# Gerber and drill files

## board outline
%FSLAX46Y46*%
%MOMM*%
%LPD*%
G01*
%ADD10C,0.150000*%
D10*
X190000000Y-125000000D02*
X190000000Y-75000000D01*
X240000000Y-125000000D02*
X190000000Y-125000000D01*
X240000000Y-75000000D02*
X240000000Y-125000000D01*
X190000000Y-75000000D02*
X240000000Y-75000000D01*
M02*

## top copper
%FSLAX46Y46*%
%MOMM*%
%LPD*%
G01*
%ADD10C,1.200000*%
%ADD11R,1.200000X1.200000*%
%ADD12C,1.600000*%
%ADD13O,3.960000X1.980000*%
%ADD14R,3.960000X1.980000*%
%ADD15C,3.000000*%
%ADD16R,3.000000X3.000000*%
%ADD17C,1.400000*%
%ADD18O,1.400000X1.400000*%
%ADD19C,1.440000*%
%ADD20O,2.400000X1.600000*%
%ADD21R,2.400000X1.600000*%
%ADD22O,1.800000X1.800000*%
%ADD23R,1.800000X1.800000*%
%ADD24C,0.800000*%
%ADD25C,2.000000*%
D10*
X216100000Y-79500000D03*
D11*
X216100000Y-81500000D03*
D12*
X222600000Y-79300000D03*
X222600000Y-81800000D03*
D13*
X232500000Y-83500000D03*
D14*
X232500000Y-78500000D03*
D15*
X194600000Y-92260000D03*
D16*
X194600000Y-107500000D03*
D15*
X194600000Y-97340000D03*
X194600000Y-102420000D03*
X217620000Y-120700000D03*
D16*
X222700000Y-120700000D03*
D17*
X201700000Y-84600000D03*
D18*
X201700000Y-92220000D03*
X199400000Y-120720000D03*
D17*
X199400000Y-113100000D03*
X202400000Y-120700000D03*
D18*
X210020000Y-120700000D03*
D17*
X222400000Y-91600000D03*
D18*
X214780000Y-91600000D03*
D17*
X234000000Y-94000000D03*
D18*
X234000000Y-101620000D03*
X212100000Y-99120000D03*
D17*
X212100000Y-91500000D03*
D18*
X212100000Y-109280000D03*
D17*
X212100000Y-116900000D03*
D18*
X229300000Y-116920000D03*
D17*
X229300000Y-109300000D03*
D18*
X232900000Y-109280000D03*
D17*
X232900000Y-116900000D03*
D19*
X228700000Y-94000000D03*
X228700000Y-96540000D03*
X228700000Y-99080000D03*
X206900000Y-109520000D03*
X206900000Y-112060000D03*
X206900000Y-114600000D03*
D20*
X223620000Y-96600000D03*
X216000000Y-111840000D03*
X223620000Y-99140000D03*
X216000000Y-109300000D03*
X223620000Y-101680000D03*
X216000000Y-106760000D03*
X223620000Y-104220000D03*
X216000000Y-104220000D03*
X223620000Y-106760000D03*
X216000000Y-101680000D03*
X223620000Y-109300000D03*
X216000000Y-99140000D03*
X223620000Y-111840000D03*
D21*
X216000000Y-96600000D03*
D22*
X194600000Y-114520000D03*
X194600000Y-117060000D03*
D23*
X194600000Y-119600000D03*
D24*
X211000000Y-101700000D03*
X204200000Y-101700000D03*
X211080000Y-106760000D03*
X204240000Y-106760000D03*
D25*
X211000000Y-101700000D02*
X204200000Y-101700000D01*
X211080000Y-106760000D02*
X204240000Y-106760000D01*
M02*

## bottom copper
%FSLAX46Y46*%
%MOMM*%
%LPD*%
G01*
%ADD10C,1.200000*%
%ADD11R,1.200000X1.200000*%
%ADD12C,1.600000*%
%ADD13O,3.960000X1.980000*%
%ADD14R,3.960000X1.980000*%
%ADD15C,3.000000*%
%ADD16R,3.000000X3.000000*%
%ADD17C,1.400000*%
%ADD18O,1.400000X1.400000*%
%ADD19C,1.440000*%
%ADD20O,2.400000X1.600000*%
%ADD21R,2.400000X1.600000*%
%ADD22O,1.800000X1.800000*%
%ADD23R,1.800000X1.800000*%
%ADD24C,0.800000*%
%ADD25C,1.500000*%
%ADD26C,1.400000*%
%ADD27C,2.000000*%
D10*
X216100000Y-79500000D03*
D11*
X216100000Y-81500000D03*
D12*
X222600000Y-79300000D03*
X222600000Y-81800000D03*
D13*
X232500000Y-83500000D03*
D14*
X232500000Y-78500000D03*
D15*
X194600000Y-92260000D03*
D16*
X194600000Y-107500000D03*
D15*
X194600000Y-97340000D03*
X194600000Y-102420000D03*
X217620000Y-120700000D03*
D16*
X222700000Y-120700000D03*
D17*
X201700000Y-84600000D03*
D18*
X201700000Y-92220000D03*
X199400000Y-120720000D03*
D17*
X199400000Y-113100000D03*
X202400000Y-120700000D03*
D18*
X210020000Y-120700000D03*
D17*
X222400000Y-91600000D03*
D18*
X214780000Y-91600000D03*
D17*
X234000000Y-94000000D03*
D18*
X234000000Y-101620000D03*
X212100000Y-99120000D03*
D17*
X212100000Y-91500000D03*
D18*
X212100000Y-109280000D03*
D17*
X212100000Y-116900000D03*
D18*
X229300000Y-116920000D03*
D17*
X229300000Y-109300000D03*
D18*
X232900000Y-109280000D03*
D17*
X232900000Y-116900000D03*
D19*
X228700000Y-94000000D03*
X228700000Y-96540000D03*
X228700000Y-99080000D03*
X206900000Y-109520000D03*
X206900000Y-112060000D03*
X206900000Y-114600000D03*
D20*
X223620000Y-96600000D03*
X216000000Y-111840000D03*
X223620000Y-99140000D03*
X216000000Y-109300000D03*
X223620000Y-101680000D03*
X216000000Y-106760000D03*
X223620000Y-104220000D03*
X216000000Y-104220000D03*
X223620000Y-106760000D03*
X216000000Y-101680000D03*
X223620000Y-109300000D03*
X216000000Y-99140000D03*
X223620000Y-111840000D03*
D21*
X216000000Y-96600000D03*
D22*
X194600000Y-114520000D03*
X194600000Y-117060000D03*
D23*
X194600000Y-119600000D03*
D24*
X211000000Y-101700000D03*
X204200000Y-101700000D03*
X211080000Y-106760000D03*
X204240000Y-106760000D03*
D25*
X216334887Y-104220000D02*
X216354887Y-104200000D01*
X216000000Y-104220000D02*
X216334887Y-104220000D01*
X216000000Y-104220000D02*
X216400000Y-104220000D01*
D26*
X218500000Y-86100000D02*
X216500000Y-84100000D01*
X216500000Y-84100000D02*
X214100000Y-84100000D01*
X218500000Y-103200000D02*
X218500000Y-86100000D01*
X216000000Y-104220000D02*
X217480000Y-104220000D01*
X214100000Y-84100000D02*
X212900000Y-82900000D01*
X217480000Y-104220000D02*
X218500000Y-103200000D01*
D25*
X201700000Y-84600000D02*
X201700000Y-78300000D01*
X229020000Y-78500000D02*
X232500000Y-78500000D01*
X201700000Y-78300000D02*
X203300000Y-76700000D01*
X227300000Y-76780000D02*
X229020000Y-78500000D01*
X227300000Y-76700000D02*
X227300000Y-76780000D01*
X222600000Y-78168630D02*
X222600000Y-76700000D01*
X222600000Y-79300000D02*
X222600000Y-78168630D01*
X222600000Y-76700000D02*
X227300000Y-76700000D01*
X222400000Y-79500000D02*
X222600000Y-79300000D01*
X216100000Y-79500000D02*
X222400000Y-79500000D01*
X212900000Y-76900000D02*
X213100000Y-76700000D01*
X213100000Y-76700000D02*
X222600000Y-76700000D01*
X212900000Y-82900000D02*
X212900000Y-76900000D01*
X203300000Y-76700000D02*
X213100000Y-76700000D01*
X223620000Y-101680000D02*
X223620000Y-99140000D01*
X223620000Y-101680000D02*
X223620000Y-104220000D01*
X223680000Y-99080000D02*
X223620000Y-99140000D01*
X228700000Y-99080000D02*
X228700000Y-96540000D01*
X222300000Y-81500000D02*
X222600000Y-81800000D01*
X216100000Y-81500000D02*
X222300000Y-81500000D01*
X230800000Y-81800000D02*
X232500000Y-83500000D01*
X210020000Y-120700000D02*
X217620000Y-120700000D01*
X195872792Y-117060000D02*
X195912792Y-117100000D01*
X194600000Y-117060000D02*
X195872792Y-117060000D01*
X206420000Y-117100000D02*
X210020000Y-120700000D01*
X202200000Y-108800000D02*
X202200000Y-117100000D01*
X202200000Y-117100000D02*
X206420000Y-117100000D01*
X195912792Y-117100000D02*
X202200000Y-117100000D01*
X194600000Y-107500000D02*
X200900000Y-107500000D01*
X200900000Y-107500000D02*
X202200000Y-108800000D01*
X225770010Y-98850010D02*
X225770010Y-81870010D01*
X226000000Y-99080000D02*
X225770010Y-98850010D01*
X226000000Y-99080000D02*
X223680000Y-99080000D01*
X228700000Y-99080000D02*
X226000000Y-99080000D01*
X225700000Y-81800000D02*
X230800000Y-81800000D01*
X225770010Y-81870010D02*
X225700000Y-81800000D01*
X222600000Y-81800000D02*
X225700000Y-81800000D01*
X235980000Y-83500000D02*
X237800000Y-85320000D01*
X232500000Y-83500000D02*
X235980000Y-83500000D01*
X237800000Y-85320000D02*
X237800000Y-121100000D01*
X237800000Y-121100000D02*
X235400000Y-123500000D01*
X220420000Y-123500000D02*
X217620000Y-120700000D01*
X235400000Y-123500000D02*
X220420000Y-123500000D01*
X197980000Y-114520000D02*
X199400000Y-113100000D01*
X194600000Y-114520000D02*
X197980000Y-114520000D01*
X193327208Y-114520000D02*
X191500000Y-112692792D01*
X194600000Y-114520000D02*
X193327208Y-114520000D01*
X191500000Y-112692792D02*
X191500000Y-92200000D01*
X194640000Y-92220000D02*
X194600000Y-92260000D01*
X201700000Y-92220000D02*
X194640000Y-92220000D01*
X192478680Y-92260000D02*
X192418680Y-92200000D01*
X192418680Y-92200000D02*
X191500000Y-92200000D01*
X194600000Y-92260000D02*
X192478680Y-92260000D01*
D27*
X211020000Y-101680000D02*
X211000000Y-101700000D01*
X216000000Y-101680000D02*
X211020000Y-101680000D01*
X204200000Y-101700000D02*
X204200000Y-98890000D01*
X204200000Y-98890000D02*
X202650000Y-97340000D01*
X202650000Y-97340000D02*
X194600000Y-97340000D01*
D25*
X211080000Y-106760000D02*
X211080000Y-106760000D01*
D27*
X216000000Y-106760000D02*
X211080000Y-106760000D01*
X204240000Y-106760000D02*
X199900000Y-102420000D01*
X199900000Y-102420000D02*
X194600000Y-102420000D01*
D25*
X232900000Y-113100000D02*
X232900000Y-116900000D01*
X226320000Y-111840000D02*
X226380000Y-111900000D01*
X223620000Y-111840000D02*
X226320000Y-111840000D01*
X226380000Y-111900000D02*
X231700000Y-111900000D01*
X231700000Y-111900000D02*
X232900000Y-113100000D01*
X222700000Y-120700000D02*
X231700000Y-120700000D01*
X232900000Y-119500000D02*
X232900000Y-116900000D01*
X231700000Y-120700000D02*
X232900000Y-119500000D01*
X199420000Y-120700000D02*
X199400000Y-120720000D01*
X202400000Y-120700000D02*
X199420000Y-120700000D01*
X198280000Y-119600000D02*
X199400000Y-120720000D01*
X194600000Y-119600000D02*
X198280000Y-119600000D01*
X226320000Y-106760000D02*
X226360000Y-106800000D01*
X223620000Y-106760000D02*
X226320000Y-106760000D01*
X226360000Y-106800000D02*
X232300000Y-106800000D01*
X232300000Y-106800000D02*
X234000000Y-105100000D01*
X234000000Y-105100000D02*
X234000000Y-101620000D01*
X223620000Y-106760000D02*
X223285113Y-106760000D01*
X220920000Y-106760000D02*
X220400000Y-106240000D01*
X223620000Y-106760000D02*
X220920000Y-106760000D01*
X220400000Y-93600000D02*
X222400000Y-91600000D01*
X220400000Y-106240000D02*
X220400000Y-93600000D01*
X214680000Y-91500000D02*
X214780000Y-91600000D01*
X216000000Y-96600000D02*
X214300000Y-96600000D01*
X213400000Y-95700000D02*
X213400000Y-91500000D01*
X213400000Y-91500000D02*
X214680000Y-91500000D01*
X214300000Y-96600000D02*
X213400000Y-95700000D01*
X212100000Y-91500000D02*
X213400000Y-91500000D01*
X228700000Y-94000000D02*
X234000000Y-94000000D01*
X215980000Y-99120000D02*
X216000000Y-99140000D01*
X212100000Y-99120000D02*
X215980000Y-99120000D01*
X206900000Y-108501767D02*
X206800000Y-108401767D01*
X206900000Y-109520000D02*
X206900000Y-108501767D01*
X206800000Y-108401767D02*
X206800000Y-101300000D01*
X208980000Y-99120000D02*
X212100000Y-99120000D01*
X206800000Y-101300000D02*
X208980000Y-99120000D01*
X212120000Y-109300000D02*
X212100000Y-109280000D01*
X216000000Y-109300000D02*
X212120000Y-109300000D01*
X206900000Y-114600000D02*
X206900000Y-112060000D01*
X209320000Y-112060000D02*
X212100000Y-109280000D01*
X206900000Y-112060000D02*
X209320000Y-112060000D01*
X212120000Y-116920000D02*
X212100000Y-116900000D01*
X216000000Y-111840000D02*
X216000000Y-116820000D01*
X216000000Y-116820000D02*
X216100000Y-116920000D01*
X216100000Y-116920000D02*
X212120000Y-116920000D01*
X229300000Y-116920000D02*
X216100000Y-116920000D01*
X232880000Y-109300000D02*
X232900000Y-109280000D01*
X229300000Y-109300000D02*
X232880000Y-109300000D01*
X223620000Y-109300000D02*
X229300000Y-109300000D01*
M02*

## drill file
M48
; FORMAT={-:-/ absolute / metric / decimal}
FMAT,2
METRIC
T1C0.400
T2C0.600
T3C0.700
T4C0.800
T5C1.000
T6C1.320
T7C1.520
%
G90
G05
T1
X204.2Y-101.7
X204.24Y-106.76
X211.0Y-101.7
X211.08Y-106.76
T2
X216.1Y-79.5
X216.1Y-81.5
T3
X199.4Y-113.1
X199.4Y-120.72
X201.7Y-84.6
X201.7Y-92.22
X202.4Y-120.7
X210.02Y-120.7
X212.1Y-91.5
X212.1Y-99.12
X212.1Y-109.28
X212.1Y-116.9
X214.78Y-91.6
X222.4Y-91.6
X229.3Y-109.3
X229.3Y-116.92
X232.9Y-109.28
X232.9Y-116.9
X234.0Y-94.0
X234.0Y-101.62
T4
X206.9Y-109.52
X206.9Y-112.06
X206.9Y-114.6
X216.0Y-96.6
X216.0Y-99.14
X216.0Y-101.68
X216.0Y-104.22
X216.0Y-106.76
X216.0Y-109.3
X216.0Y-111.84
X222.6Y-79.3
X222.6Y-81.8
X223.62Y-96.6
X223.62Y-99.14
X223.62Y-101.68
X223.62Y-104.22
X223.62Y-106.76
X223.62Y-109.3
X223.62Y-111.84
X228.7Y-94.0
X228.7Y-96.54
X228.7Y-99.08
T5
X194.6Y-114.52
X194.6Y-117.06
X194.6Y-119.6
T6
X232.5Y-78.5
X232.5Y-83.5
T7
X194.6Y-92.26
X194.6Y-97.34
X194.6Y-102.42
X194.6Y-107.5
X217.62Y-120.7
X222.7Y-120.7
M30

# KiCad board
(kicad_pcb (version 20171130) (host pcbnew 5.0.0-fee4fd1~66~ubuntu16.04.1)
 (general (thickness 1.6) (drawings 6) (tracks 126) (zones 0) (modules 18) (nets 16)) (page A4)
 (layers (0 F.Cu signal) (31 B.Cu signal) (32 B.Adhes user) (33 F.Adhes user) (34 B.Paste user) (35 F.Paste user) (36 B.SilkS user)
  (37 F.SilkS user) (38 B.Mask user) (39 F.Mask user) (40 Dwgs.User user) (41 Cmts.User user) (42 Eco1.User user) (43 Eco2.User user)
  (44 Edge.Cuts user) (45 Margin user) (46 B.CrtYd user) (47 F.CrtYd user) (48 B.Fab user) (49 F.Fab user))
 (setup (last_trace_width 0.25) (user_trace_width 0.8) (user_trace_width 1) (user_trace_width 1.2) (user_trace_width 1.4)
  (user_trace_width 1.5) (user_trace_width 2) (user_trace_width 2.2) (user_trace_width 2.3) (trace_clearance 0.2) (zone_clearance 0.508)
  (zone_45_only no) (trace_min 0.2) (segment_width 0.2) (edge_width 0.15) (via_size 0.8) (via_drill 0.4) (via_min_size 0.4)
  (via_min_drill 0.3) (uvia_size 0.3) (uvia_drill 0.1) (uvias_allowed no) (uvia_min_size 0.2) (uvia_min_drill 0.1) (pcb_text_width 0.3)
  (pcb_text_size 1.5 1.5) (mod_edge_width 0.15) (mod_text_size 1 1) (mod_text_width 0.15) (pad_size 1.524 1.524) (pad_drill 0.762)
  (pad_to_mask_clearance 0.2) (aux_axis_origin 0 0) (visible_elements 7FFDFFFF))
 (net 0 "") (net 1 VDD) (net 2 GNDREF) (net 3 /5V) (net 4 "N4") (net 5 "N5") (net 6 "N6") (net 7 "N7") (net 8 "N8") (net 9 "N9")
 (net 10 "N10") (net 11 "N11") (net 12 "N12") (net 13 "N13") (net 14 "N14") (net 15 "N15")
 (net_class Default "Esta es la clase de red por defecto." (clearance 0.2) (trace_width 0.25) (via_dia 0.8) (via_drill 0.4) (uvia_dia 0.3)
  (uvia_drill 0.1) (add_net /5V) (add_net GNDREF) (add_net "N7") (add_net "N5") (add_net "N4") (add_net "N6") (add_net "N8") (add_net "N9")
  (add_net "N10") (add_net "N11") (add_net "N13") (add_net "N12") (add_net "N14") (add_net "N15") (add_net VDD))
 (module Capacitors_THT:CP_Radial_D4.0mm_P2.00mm (layer F.Cu) (at 216.1 81.5 90)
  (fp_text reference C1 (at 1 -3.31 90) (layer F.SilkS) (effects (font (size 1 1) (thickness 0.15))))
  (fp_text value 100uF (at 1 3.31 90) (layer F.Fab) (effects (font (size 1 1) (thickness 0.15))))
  (pad 2 thru_hole circle (at 2 0 90) (size 1.2 1.2) (drill 0.6) (layers *.Cu *.Mask) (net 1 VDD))
  (pad 1 thru_hole rect (at 0 0 90) (size 1.2 1.2) (drill 0.6) (layers *.Cu *.Mask) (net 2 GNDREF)))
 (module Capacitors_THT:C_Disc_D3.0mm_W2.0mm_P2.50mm (layer F.Cu) (at 222.6 81.8 90)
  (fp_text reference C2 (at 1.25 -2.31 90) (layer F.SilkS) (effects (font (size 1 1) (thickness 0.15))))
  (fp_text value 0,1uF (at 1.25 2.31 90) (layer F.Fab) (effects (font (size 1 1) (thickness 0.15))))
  (pad 2 thru_hole circle (at 2.5 0 90) (size 1.6 1.6) (drill 0.8) (layers *.Cu *.Mask) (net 1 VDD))
  (pad 1 thru_hole circle (at 0 0 90) (size 1.6 1.6) (drill 0.8) (layers *.Cu *.Mask) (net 2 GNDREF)))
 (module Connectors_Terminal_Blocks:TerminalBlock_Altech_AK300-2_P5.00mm (layer F.Cu) (at 232.5 78.5 270)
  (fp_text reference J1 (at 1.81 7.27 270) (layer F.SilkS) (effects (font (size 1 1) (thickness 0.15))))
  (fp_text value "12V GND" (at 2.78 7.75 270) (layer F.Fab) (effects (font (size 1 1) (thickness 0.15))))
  (pad 2 thru_hole oval (at 5 0 270) (size 1.98 3.96) (drill 1.32) (layers *.Cu *.Mask) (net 2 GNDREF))
  (pad 1 thru_hole rect (at 0 0 270) (size 1.98 3.96) (drill 1.32) (layers *.Cu *.Mask) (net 1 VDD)))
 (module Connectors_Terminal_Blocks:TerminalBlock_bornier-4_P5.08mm (layer F.Cu) (at 194.6 107.5 90)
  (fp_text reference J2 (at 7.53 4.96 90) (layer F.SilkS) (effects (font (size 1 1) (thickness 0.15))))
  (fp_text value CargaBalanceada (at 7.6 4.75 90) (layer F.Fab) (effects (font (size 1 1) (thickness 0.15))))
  (pad 4 thru_hole circle (at 15.24 0 90) (size 3 3) (drill 1.52) (layers *.Cu *.Mask) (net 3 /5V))
  (pad 1 thru_hole rect (at 0 0 90) (size 3 3) (drill 1.52) (layers *.Cu *.Mask) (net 2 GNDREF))
  (pad 3 thru_hole circle (at 10.16 0 90) (size 3 3) (drill 1.52) (layers *.Cu *.Mask) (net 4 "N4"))
  (pad 2 thru_hole circle (at 5.08 0 90) (size 3 3) (drill 1.52) (layers *.Cu *.Mask) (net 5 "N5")))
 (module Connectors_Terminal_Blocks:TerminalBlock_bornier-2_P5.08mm (layer F.Cu) (at 222.7 120.7 180)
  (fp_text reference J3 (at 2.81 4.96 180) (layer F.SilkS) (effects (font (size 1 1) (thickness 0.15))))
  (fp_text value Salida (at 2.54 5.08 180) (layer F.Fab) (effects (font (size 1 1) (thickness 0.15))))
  (pad 2 thru_hole circle (at 5.08 0 180) (size 3 3) (drill 1.52) (layers *.Cu *.Mask) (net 2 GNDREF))
  (pad 1 thru_hole rect (at 0 0 180) (size 3 3) (drill 1.52) (layers *.Cu *.Mask) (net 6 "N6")))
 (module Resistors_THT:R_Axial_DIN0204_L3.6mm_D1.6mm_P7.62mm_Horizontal (layer F.Cu) (at 201.7 84.6 270)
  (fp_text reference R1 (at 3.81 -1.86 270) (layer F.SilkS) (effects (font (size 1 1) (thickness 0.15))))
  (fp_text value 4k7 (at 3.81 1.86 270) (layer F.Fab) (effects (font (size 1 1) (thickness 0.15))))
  (pad 1 thru_hole circle (at 0 0 270) (size 1.4 1.4) (drill 0.7) (layers *.Cu *.Mask) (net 1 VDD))
  (pad 2 thru_hole oval (at 7.62 0 270) (size 1.4 1.4) (drill 0.7) (layers *.Cu *.Mask) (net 3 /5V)))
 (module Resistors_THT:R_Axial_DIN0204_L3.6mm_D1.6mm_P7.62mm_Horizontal (layer F.Cu) (at 199.4 113.1 270)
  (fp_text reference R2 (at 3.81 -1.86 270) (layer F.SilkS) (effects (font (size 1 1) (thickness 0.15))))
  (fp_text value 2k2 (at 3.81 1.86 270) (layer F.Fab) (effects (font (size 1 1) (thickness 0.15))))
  (pad 2 thru_hole oval (at 7.62 0 270) (size 1.4 1.4) (drill 0.7) (layers *.Cu *.Mask) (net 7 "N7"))
  (pad 1 thru_hole circle (at 0 0 270) (size 1.4 1.4) (drill 0.7) (layers *.Cu *.Mask) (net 3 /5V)))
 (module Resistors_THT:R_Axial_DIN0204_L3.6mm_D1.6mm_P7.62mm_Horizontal (layer F.Cu) (at 202.4 120.7)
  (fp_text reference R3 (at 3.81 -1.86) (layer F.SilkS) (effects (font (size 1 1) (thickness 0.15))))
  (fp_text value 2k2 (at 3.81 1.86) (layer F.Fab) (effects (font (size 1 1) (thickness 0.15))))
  (pad 1 thru_hole circle (at 0 0) (size 1.4 1.4) (drill 0.7) (layers *.Cu *.Mask) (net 7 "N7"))
  (pad 2 thru_hole oval (at 7.62 0) (size 1.4 1.4) (drill 0.7) (layers *.Cu *.Mask) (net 2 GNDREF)))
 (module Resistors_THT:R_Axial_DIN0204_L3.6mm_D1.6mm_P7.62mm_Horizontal (layer F.Cu) (at 222.4 91.6 180)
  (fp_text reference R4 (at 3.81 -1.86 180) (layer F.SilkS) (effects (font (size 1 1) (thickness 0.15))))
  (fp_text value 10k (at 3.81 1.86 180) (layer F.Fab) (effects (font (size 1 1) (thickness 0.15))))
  (pad 1 thru_hole circle (at 0 0 180) (size 1.4 1.4) (drill 0.7) (layers *.Cu *.Mask) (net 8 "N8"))
  (pad 2 thru_hole oval (at 7.62 0 180) (size 1.4 1.4) (drill 0.7) (layers *.Cu *.Mask) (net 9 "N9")))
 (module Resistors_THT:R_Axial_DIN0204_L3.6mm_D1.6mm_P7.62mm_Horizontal (layer F.Cu) (at 234 94 270)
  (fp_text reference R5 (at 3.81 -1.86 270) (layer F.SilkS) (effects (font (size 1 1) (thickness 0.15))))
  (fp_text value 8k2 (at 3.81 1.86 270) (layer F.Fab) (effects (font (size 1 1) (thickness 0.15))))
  (pad 1 thru_hole circle (at 0 0 270) (size 1.4 1.4) (drill 0.7) (layers *.Cu *.Mask) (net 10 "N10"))
  (pad 2 thru_hole oval (at 7.62 0 270) (size 1.4 1.4) (drill 0.7) (layers *.Cu *.Mask) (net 8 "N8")))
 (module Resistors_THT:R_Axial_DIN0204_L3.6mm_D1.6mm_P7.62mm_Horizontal (layer F.Cu) (at 212.1 91.5 270)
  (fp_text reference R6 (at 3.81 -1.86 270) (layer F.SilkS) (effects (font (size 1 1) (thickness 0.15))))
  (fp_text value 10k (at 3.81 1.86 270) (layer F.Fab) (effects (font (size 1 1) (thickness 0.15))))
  (pad 2 thru_hole oval (at 7.62 0 270) (size 1.4 1.4) (drill 0.7) (layers *.Cu *.Mask) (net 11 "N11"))
  (pad 1 thru_hole circle (at 0 0 270) (size 1.4 1.4) (drill 0.7) (layers *.Cu *.Mask) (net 9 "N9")))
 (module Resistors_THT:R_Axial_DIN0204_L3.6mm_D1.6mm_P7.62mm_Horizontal (layer F.Cu) (at 212.1 116.9 90)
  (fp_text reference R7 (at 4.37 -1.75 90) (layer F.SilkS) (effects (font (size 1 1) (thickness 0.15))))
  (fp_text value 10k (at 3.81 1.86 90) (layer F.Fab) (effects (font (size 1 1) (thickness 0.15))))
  (pad 2 thru_hole oval (at 7.62 0 90) (size 1.4 1.4) (drill 0.7) (layers *.Cu *.Mask) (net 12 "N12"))
  (pad 1 thru_hole circle (at 0 0 90) (size 1.4 1.4) (drill 0.7) (layers *.Cu *.Mask) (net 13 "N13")))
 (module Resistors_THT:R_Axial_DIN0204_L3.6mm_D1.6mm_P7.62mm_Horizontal (layer F.Cu) (at 229.3 109.3 270)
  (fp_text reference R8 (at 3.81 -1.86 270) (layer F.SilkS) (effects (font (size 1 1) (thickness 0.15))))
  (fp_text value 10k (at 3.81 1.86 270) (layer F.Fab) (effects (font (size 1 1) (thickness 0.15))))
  (pad 2 thru_hole oval (at 7.62 0 270) (size 1.4 1.4) (drill 0.7) (layers *.Cu *.Mask) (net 13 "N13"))
  (pad 1 thru_hole circle (at 0 0 270) (size 1.4 1.4) (drill 0.7) (layers *.Cu *.Mask) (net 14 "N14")))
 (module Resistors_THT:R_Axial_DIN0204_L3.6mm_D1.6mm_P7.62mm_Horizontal (layer F.Cu) (at 232.9 116.9 90)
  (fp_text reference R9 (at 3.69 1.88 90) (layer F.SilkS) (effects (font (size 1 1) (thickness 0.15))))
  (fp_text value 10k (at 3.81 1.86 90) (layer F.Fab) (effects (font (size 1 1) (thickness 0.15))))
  (pad 2 thru_hole oval (at 7.62 0 90) (size 1.4 1.4) (drill 0.7) (layers *.Cu *.Mask) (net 14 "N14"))
  (pad 1 thru_hole circle (at 0 0 90) (size 1.4 1.4) (drill 0.7) (layers *.Cu *.Mask) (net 6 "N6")))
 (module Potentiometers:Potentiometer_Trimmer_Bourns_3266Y (layer F.Cu) (at 228.7 94 90)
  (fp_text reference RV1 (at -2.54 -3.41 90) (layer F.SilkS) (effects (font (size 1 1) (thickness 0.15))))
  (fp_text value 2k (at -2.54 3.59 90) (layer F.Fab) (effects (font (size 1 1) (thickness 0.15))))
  (pad 1 thru_hole circle (at 0 0 90) (size 1.44 1.44) (drill 0.8) (layers *.Cu *.Mask) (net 10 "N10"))
  (pad 2 thru_hole circle (at -2.54 0 90) (size 1.44 1.44) (drill 0.8) (layers *.Cu *.Mask) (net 2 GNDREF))
  (pad 3 thru_hole circle (at -5.08 0 90) (size 1.44 1.44) (drill 0.8) (layers *.Cu *.Mask) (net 2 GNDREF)))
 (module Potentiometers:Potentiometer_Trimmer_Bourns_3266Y (layer F.Cu) (at 206.9 114.6 270)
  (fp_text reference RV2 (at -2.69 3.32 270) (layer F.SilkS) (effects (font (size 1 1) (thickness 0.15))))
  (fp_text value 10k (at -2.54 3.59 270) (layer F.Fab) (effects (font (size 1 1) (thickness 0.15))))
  (pad 3 thru_hole circle (at -5.08 0 270) (size 1.44 1.44) (drill 0.8) (layers *.Cu *.Mask) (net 11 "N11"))
  (pad 2 thru_hole circle (at -2.54 0 270) (size 1.44 1.44) (drill 0.8) (layers *.Cu *.Mask) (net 12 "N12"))
  (pad 1 thru_hole circle (at 0 0 270) (size 1.44 1.44) (drill 0.8) (layers *.Cu *.Mask) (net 12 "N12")))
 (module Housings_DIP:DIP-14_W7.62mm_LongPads (layer F.Cu) (at 216 96.6)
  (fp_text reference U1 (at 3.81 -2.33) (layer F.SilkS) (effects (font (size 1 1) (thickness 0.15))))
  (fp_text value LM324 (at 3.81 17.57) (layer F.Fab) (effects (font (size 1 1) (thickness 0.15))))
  (pad 14 thru_hole oval (at 7.62 0) (size 2.4 1.6) (drill 0.8) (layers *.Cu *.Mask) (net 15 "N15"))
  (pad 7 thru_hole oval (at 0 15.24) (size 2.4 1.6) (drill 0.8) (layers *.Cu *.Mask) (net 13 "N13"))
  (pad 13 thru_hole oval (at 7.62 2.54) (size 2.4 1.6) (drill 0.8) (layers *.Cu *.Mask) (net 2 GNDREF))
  (pad 6 thru_hole oval (at 0 12.7) (size 2.4 1.6) (drill 0.8) (layers *.Cu *.Mask) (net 12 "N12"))
  (pad 12 thru_hole oval (at 7.62 5.08) (size 2.4 1.6) (drill 0.8) (layers *.Cu *.Mask) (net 2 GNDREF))
  (pad 5 thru_hole oval (at 0 10.16) (size 2.4 1.6) (drill 0.8) (layers *.Cu *.Mask) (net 5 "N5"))
  (pad 11 thru_hole oval (at 7.62 7.62) (size 2.4 1.6) (drill 0.8) (layers *.Cu *.Mask) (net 2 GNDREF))
  (pad 4 thru_hole oval (at 0 7.62) (size 2.4 1.6) (drill 0.8) (layers *.Cu *.Mask) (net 1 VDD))
  (pad 10 thru_hole oval (at 7.62 10.16) (size 2.4 1.6) (drill 0.8) (layers *.Cu *.Mask) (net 8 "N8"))
  (pad 3 thru_hole oval (at 0 5.08) (size 2.4 1.6) (drill 0.8) (layers *.Cu *.Mask) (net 4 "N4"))
  (pad 9 thru_hole oval (at 7.62 12.7) (size 2.4 1.6) (drill 0.8) (layers *.Cu *.Mask) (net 14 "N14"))
  (pad 2 thru_hole oval (at 0 2.54) (size 2.4 1.6) (drill 0.8) (layers *.Cu *.Mask) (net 11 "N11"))
  (pad 8 thru_hole oval (at 7.62 15.24) (size 2.4 1.6) (drill 0.8) (layers *.Cu *.Mask) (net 6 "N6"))
  (pad 1 thru_hole rect (at 0 0) (size 2.4 1.6) (drill 0.8) (layers *.Cu *.Mask) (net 9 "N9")))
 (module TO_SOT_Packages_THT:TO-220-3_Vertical (layer F.Cu) (at 194.6 119.6 90)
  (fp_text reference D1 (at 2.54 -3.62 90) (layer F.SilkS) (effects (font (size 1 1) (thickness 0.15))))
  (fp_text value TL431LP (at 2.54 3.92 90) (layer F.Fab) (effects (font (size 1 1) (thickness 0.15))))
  (pad 3 thru_hole oval (at 5.08 0 90) (size 1.8 1.8) (drill 1) (layers *.Cu *.Mask) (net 3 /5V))
  (pad 2 thru_hole oval (at 2.54 0 90) (size 1.8 1.8) (drill 1) (layers *.Cu *.Mask) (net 2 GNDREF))
  (pad 1 thru_hole rect (at 0 0 90) (size 1.8 1.8) (drill 1) (layers *.Cu *.Mask) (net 7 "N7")))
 (gr_line (start 190 125) (end 190 75) (layer Edge.Cuts) (width 0.15))
 (gr_line (start 240 125) (end 190 125) (layer Edge.Cuts) (width 0.15))
 (gr_line (start 240 75) (end 240 125) (layer Edge.Cuts) (width 0.15))
 (gr_line (start 190 75) (end 240 75) (layer Edge.Cuts) (width 0.15))
 (segment (start 216.334887 104.22) (end 216.354887 104.2) (width 1.5) (layer B.Cu) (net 1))
 (segment (start 216 104.22) (end 216.334887 104.22) (width 1.5) (layer B.Cu) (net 1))
 (segment (start 216 104.22) (end 216.4 104.22) (width 1.5) (layer B.Cu) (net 1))
 (segment (start 218.5 86.1) (end 216.5 84.1) (width 1.4) (layer B.Cu) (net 1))
 (segment (start 216.5 84.1) (end 214.1 84.1) (width 1.4) (layer B.Cu) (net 1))
 (segment (start 218.5 103.2) (end 218.5 86.1) (width 1.4) (layer B.Cu) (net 1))
 (segment (start 216 104.22) (end 217.48 104.22) (width 1.4) (layer B.Cu) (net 1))
 (segment (start 214.1 84.1) (end 212.9 82.9) (width 1.4) (layer B.Cu) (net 1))
 (segment (start 217.48 104.22) (end 218.5 103.2) (width 1.4) (layer B.Cu) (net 1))
 (segment (start 201.7 84.6) (end 201.7 78.3) (width 1.5) (layer B.Cu) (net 1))
 (segment (start 229.02 78.5) (end 232.5 78.5) (width 1.5) (layer B.Cu) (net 1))
 (segment (start 201.7 78.3) (end 203.3 76.7) (width 1.5) (layer B.Cu) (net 1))
 (segment (start 227.3 76.78) (end 229.02 78.5) (width 1.5) (layer B.Cu) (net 1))
 (segment (start 227.3 76.7) (end 227.3 76.78) (width 1.5) (layer B.Cu) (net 1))
 (segment (start 222.6 78.16863) (end 222.6 76.7) (width 1.5) (layer B.Cu) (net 1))
 (segment (start 222.6 79.3) (end 222.6 78.16863) (width 1.5) (layer B.Cu) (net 1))
 (segment (start 222.6 76.7) (end 227.3 76.7) (width 1.5) (layer B.Cu) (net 1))
 (segment (start 222.4 79.5) (end 222.6 79.3) (width 1.5) (layer B.Cu) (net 1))
 (segment (start 216.1 79.5) (end 222.4 79.5) (width 1.5) (layer B.Cu) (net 1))
 (segment (start 212.9 76.9) (end 213.1 76.7) (width 1.5) (layer B.Cu) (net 1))
 (segment (start 213.1 76.7) (end 222.6 76.7) (width 1.5) (layer B.Cu) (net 1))
 (segment (start 212.9 82.9) (end 212.9 76.9) (width 1.5) (layer B.Cu) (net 1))
 (segment (start 203.3 76.7) (end 213.1 76.7) (width 1.5) (layer B.Cu) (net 1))
 (segment (start 223.62 101.68) (end 223.62 99.14) (width 1.5) (layer B.Cu) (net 2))
 (segment (start 223.62 101.68) (end 223.62 104.22) (width 1.5) (layer B.Cu) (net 2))
 (segment (start 223.68 99.08) (end 223.62 99.14) (width 1.5) (layer B.Cu) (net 2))
 (segment (start 228.7 99.08) (end 228.7 96.54) (width 1.5) (layer B.Cu) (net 2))
 (segment (start 222.3 81.5) (end 222.6 81.8) (width 1.5) (layer B.Cu) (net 2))
 (segment (start 216.1 81.5) (end 222.3 81.5) (width 1.5) (layer B.Cu) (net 2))
 (segment (start 230.8 81.8) (end 232.5 83.5) (width 1.5) (layer B.Cu) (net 2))
 (segment (start 210.02 120.7) (end 217.62 120.7) (width 1.5) (layer B.Cu) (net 2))
 (segment (start 195.872792 117.06) (end 195.912792 117.1) (width 1.5) (layer B.Cu) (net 2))
 (segment (start 194.6 117.06) (end 195.872792 117.06) (width 1.5) (layer B.Cu) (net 2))
 (segment (start 206.42 117.1) (end 210.02 120.7) (width 1.5) (layer B.Cu) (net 2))
 (segment (start 202.2 108.8) (end 202.2 117.1) (width 1.5) (layer B.Cu) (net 2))
 (segment (start 202.2 117.1) (end 206.42 117.1) (width 1.5) (layer B.Cu) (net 2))
 (segment (start 195.912792 117.1) (end 202.2 117.1) (width 1.5) (layer B.Cu) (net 2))
 (segment (start 194.6 107.5) (end 200.9 107.5) (width 1.5) (layer B.Cu) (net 2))
 (segment (start 200.9 107.5) (end 202.2 108.8) (width 1.5) (layer B.Cu) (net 2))
 (segment (start 225.77001 98.85001) (end 225.77001 81.87001) (width 1.5) (layer B.Cu) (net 2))
 (segment (start 226 99.08) (end 225.77001 98.85001) (width 1.5) (layer B.Cu) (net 2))
 (segment (start 226 99.08) (end 223.68 99.08) (width 1.5) (layer B.Cu) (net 2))
 (segment (start 228.7 99.08) (end 226 99.08) (width 1.5) (layer B.Cu) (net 2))
 (segment (start 225.7 81.8) (end 230.8 81.8) (width 1.5) (layer B.Cu) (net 2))
 (segment (start 225.77001 81.87001) (end 225.7 81.8) (width 1.5) (layer B.Cu) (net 2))
 (segment (start 222.6 81.8) (end 225.7 81.8) (width 1.5) (layer B.Cu) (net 2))
 (segment (start 235.98 83.5) (end 237.8 85.32) (width 1.5) (layer B.Cu) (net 2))
 (segment (start 232.5 83.5) (end 235.98 83.5) (width 1.5) (layer B.Cu) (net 2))
 (segment (start 237.8 85.32) (end 237.8 121.1) (width 1.5) (layer B.Cu) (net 2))
 (segment (start 237.8 121.1) (end 235.4 123.5) (width 1.5) (layer B.Cu) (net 2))
 (segment (start 220.42 123.5) (end 217.62 120.7) (width 1.5) (layer B.Cu) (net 2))
 (segment (start 235.4 123.5) (end 220.42 123.5) (width 1.5) (layer B.Cu) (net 2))
 (segment (start 197.98 114.52) (end 199.4 113.1) (width 1.5) (layer B.Cu) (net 3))
 (segment (start 194.6 114.52) (end 197.98 114.52) (width 1.5) (layer B.Cu) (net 3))
 (segment (start 193.327208 114.52) (end 191.5 112.692792) (width 1.5) (layer B.Cu) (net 3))
 (segment (start 194.6 114.52) (end 193.327208 114.52) (width 1.5) (layer B.Cu) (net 3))
 (segment (start 191.5 112.692792) (end 191.5 92.2) (width 1.5) (layer B.Cu) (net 3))
 (segment (start 194.64 92.22) (end 194.6 92.26) (width 1.5) (layer B.Cu) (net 3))
 (segment (start 201.7 92.22) (end 194.64 92.22) (width 1.5) (layer B.Cu) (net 3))
 (segment (start 192.47868 92.26) (end 192.41868 92.2) (width 1.5) (layer B.Cu) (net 3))
 (segment (start 192.41868 92.2) (end 191.5 92.2) (width 1.5) (layer B.Cu) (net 3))
 (segment (start 194.6 92.26) (end 192.47868 92.26) (width 1.5) (layer B.Cu) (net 3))
 (via (at 211 101.7) (size 0.8) (drill 0.4) (layers F.Cu B.Cu) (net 4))
 (via (at 204.2 101.7) (size 0.8) (drill 0.4) (layers F.Cu B.Cu) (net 4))
 (segment (start 211.02 101.68) (end 211 101.7) (width 2) (layer B.Cu) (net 4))
 (segment (start 216 101.68) (end 211.02 101.68) (width 2) (layer B.Cu) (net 4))
 (segment (start 204.2 101.7) (end 204.2 98.89) (width 2) (layer B.Cu) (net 4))
 (segment (start 204.2 98.89) (end 202.65 97.34) (width 2) (layer B.Cu) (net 4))
 (segment (start 202.65 97.34) (end 194.6 97.34) (width 2) (layer B.Cu) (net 4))
 (segment (start 211 101.7) (end 204.2 101.7) (width 2) (layer F.Cu) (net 4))
 (segment (start 211.08 106.76) (end 211.08 106.76) (width 1.5) (layer B.Cu) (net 5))
 (via (at 211.08 106.76) (size 0.8) (drill 0.4) (layers F.Cu B.Cu) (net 5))
 (via (at 204.24 106.76) (size 0.8) (drill 0.4) (layers F.Cu B.Cu) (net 5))
 (segment (start 216 106.76) (end 211.08 106.76) (width 2) (layer B.Cu) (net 5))
 (segment (start 204.24 106.76) (end 199.9 102.42) (width 2) (layer B.Cu) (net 5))
 (segment (start 199.9 102.42) (end 194.6 102.42) (width 2) (layer B.Cu) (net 5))
 (segment (start 211.08 106.76) (end 204.24 106.76) (width 2) (layer F.Cu) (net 5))
 (segment (start 232.9 113.1) (end 232.9 116.9) (width 1.5) (layer B.Cu) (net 6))
 (segment (start 226.32 111.84) (end 226.38 111.9) (width 1.5) (layer B.Cu) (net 6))
 (segment (start 223.62 111.84) (end 226.32 111.84) (width 1.5) (layer B.Cu) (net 6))
 (segment (start 226.38 111.9) (end 231.7 111.9) (width 1.5) (layer B.Cu) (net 6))
 (segment (start 231.7 111.9) (end 232.9 113.1) (width 1.5) (layer B.Cu) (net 6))
 (segment (start 222.7 120.7) (end 231.7 120.7) (width 1.5) (layer B.Cu) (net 6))
 (segment (start 232.9 119.5) (end 232.9 116.9) (width 1.5) (layer B.Cu) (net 6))
 (segment (start 231.7 120.7) (end 232.9 119.5) (width 1.5) (layer B.Cu) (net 6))
 (segment (start 199.42 120.7) (end 199.4 120.72) (width 1.5) (layer B.Cu) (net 7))
 (segment (start 202.4 120.7) (end 199.42 120.7) (width 1.5) (layer B.Cu) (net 7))
 (segment (start 198.28 119.6) (end 199.4 120.72) (width 1.5) (layer B.Cu) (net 7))
 (segment (start 194.6 119.6) (end 198.28 119.6) (width 1.5) (layer B.Cu) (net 7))
 (segment (start 226.32 106.76) (end 226.36 106.8) (width 1.5) (layer B.Cu) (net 8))
 (segment (start 223.62 106.76) (end 226.32 106.76) (width 1.5) (layer B.Cu) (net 8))
 (segment (start 226.36 106.8) (end 232.3 106.8) (width 1.5) (layer B.Cu) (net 8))
 (segment (start 232.3 106.8) (end 234 105.1) (width 1.5) (layer B.Cu) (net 8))
 (segment (start 234 105.1) (end 234 101.62) (width 1.5) (layer B.Cu) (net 8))
 (segment (start 223.62 106.76) (end 223.285113 106.76) (width 1.5) (layer B.Cu) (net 8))
 (segment (start 220.92 106.76) (end 220.4 106.24) (width 1.5) (layer B.Cu) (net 8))
 (segment (start 223.62 106.76) (end 220.92 106.76) (width 1.5) (layer B.Cu) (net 8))
 (segment (start 220.4 93.6) (end 222.4 91.6) (width 1.5) (layer B.Cu) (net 8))
 (segment (start 220.4 106.24) (end 220.4 93.6) (width 1.5) (layer B.Cu) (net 8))
 (segment (start 214.68 91.5) (end 214.78 91.6) (width 1.5) (layer B.Cu) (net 9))
 (segment (start 216 96.6) (end 214.3 96.6) (width 1.5) (layer B.Cu) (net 9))
 (segment (start 213.4 95.7) (end 213.4 91.5) (width 1.5) (layer B.Cu) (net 9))
 (segment (start 213.4 91.5) (end 214.68 91.5) (width 1.5) (layer B.Cu) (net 9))
 (segment (start 214.3 96.6) (end 213.4 95.7) (width 1.5) (layer B.Cu) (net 9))
 (segment (start 212.1 91.5) (end 213.4 91.5) (width 1.5) (layer B.Cu) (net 9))
 (segment (start 228.7 94) (end 234 94) (width 1.5) (layer B.Cu) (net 10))
 (segment (start 215.98 99.12) (end 216 99.14) (width 1.5) (layer B.Cu) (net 11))
 (segment (start 212.1 99.12) (end 215.98 99.12) (width 1.5) (layer B.Cu) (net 11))
 (segment (start 206.9 108.501767) (end 206.8 108.401767) (width 1.5) (layer B.Cu) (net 11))
 (segment (start 206.9 109.52) (end 206.9 108.501767) (width 1.5) (layer B.Cu) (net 11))
 (segment (start 206.8 108.401767) (end 206.8 101.3) (width 1.5) (layer B.Cu) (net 11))
 (segment (start 208.98 99.12) (end 212.1 99.12) (width 1.5) (layer B.Cu) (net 11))
 (segment (start 206.8 101.3) (end 208.98 99.12) (width 1.5) (layer B.Cu) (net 11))
 (segment (start 212.12 109.3) (end 212.1 109.28) (width 1.5) (layer B.Cu) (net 12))
 (segment (start 216 109.3) (end 212.12 109.3) (width 1.5) (layer B.Cu) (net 12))
 (segment (start 206.9 114.6) (end 206.9 112.06) (width 1.5) (layer B.Cu) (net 12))
 (segment (start 209.32 112.06) (end 212.1 109.28) (width 1.5) (layer B.Cu) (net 12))
 (segment (start 206.9 112.06) (end 209.32 112.06) (width 1.5) (layer B.Cu) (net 12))
 (segment (start 212.12 116.92) (end 212.1 116.9) (width 1.5) (layer B.Cu) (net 13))
 (segment (start 216 111.84) (end 216 116.82) (width 1.5) (layer B.Cu) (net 13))
 (segment (start 216 116.82) (end 216.1 116.92) (width 1.5) (layer B.Cu) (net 13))
 (segment (start 216.1 116.92) (end 212.12 116.92) (width 1.5) (layer B.Cu) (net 13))
 (segment (start 229.3 116.92) (end 216.1 116.92) (width 1.5) (layer B.Cu) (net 13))
 (segment (start 232.88 109.3) (end 232.9 109.28) (width 1.5) (layer B.Cu) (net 14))
 (segment (start 229.3 109.3) (end 232.88 109.3) (width 1.5) (layer B.Cu) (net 14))
 (segment (start 223.62 109.3) (end 229.3 109.3) (width 1.5) (layer B.Cu) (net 14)))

